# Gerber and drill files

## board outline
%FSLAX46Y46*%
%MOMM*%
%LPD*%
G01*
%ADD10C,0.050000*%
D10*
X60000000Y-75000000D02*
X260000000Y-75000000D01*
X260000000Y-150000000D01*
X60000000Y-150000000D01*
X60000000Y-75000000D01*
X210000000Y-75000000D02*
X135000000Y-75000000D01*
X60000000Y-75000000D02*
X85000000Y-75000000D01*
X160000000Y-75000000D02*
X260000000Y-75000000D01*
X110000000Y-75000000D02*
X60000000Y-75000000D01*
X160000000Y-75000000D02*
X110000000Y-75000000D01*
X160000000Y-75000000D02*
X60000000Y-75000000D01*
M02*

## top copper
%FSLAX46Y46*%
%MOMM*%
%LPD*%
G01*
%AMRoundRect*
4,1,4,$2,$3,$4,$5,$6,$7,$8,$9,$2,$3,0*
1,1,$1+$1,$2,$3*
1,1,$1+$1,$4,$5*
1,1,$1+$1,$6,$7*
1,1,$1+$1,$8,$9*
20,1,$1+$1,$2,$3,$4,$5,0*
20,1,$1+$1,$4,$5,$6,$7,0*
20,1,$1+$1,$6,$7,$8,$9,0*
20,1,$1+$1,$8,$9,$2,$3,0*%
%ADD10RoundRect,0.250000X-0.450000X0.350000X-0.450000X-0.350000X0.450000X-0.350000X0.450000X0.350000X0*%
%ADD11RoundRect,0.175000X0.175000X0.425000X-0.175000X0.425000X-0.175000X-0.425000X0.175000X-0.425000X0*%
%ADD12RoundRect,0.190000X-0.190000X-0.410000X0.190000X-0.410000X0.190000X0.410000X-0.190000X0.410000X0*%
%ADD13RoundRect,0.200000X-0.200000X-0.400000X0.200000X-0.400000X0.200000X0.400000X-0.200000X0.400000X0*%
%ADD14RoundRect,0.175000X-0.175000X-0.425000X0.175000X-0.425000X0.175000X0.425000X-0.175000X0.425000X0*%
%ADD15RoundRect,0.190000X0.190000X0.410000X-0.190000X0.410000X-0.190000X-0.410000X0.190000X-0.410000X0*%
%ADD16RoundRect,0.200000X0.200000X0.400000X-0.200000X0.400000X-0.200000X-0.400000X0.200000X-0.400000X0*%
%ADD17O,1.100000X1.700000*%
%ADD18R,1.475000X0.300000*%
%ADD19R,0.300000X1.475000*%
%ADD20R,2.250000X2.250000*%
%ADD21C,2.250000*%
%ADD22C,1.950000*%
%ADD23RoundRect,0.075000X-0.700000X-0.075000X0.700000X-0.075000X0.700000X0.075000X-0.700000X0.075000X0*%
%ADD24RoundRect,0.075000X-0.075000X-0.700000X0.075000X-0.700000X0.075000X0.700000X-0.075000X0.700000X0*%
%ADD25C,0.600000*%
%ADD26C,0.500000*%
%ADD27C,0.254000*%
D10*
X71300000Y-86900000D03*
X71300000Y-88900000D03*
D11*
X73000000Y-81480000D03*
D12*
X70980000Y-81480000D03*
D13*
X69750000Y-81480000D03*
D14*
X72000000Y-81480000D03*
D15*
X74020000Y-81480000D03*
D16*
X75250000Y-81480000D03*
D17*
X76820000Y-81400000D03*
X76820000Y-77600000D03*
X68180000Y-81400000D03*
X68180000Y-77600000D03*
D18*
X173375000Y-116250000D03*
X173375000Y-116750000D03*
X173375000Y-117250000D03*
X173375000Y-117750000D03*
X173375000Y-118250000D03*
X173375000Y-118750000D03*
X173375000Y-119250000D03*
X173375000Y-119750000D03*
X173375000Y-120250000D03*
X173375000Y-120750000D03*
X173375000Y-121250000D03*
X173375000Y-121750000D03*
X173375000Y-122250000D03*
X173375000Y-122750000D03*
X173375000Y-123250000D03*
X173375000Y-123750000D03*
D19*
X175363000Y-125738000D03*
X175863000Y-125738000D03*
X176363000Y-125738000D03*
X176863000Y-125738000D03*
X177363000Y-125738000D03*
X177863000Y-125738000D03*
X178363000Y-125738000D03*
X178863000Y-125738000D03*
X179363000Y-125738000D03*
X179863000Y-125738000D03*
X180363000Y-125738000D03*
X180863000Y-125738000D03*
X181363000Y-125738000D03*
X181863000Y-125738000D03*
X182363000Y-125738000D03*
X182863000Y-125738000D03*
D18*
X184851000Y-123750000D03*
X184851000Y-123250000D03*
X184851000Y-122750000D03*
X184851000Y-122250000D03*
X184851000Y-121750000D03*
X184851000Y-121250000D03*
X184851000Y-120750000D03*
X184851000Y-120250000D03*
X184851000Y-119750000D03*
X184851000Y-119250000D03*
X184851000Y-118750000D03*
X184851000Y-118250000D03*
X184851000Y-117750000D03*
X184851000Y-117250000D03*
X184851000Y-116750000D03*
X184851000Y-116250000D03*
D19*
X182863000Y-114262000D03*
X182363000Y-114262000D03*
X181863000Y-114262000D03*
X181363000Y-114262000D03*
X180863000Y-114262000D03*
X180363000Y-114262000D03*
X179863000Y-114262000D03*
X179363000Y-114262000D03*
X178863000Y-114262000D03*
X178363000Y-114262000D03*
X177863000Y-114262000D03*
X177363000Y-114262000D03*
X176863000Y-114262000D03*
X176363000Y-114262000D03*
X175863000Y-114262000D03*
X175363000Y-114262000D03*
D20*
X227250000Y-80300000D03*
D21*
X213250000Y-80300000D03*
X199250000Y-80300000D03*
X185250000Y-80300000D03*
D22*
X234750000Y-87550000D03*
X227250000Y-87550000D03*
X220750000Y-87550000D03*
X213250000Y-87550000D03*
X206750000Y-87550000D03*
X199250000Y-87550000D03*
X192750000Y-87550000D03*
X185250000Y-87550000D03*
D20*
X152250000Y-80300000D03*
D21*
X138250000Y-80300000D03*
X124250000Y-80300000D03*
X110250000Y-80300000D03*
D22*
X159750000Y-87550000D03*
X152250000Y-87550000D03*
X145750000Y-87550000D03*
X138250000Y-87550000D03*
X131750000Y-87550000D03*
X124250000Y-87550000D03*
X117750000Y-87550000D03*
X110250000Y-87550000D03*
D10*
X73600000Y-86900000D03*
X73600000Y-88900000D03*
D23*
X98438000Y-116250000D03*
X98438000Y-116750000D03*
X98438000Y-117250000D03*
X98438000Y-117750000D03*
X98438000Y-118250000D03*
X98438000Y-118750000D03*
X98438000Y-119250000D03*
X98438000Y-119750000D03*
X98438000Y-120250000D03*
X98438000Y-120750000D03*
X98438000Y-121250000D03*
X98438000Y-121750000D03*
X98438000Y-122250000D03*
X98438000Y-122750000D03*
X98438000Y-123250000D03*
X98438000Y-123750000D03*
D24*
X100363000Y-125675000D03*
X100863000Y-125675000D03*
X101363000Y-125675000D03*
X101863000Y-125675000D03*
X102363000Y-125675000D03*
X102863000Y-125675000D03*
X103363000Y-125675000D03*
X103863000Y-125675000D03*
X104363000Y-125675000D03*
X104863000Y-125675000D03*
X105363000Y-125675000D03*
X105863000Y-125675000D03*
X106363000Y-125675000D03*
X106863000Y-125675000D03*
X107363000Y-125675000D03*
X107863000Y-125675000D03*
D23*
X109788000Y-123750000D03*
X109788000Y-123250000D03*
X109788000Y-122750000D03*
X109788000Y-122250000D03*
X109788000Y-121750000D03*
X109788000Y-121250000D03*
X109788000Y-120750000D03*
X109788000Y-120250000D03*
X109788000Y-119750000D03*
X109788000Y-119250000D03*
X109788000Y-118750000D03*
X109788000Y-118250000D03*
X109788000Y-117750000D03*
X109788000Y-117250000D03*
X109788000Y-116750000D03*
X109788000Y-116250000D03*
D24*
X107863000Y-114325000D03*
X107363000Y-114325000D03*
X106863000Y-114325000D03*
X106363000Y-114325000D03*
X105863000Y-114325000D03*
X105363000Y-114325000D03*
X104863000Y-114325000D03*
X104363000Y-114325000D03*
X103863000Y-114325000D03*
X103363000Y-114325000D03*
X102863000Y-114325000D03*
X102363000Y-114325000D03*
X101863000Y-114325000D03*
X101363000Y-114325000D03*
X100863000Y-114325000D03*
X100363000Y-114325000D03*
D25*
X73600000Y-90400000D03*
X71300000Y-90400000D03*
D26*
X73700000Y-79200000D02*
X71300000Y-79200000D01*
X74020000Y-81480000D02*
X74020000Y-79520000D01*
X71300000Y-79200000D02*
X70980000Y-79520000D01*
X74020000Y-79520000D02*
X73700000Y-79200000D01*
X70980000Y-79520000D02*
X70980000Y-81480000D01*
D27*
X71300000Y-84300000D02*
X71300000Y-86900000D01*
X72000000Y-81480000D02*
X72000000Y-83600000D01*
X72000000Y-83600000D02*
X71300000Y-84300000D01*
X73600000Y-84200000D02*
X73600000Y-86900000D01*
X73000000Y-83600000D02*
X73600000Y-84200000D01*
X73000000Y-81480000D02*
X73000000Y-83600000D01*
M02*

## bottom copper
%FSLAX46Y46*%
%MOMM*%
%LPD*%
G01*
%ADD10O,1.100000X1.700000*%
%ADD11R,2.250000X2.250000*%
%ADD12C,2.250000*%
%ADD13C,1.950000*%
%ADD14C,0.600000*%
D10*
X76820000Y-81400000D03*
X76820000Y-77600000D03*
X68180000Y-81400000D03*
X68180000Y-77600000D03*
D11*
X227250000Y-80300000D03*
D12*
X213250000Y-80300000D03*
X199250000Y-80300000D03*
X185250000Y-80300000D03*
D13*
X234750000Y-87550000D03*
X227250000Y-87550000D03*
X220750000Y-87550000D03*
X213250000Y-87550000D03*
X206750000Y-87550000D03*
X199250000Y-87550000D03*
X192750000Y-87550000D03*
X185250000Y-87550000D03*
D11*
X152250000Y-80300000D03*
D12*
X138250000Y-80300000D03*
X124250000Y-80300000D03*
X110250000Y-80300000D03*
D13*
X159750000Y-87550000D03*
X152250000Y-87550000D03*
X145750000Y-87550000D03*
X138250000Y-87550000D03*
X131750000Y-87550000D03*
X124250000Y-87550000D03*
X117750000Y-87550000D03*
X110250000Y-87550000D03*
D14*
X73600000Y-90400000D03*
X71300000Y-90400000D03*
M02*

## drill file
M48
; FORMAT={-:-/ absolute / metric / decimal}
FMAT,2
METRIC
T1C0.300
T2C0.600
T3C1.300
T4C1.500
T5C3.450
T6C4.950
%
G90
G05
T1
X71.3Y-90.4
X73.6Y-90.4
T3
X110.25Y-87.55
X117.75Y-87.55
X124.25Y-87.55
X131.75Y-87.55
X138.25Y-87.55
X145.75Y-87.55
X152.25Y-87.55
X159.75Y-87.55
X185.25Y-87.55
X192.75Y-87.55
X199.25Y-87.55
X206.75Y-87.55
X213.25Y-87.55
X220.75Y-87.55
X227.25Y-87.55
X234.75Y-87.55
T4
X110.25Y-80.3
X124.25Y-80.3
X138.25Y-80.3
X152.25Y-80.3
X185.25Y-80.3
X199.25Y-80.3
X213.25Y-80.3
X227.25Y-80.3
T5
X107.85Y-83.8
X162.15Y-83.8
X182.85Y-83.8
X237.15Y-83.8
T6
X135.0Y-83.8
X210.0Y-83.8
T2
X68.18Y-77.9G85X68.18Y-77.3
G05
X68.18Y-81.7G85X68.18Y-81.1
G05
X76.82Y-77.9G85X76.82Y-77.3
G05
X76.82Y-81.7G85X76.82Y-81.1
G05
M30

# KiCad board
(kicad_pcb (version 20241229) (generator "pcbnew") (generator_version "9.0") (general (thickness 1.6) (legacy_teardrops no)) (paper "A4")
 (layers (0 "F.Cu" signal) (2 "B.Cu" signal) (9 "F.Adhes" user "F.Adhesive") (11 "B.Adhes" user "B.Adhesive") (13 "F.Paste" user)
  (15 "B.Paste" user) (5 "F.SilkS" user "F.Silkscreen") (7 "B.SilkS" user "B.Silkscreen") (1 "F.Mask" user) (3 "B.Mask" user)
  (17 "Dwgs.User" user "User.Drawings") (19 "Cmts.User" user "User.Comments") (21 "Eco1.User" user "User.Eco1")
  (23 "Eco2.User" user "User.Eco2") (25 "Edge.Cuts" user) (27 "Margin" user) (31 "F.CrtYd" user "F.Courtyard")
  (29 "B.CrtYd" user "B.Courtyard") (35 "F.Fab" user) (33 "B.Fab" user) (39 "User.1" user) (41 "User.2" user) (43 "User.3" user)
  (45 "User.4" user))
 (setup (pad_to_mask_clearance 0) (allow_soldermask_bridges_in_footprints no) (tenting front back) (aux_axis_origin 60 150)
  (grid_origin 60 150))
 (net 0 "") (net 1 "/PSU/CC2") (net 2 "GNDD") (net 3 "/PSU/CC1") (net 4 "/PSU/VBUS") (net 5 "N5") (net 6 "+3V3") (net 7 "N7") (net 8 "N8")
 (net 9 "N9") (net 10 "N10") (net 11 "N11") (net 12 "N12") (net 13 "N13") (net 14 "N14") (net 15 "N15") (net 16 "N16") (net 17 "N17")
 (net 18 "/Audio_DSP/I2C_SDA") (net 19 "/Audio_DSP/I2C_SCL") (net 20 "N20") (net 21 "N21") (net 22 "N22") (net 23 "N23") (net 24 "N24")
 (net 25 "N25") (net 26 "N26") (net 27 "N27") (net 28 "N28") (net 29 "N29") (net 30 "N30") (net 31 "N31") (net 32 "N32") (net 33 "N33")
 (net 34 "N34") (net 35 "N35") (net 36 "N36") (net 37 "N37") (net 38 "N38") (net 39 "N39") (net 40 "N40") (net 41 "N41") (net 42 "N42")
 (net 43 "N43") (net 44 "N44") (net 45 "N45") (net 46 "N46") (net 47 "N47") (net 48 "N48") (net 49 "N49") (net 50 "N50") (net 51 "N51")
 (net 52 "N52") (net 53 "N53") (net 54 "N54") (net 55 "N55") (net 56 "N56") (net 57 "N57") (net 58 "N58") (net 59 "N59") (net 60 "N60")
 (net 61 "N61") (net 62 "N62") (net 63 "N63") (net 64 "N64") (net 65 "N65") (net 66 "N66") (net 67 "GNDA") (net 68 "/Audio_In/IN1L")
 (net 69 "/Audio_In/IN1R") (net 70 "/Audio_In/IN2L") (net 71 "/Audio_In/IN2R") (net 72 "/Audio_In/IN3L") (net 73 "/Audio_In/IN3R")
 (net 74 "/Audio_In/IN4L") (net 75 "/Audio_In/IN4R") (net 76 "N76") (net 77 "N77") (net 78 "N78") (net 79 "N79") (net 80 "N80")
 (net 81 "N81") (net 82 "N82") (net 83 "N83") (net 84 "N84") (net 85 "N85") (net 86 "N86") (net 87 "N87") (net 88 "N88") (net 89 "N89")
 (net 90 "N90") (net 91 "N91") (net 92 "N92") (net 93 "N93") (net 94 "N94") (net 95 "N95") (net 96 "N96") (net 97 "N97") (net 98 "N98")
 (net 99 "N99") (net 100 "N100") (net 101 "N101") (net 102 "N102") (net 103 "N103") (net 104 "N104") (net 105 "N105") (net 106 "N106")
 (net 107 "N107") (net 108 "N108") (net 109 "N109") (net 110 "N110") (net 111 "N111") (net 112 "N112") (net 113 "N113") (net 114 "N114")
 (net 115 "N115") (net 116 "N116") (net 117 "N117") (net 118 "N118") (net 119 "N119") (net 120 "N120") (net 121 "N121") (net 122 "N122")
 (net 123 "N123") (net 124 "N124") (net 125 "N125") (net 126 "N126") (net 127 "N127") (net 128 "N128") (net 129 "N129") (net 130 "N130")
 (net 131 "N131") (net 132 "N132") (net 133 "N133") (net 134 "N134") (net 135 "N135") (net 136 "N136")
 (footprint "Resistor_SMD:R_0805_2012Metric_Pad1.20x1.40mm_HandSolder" (layer "F.Cu") (at 71.3 87.9 -90)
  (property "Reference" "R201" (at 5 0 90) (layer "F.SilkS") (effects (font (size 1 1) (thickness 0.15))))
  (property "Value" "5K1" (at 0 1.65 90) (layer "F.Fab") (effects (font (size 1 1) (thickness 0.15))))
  (pad "1" smd roundrect (at -1 0 270) (size 1.2 1.4) (layers "F.Cu" "F.Mask" "F.Paste") (roundrect_rratio 0.208333) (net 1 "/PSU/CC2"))
  (pad "2" smd roundrect (at 1 0 270) (size 1.2 1.4) (layers "F.Cu" "F.Mask" "F.Paste") (roundrect_rratio 0.208333) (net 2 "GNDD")))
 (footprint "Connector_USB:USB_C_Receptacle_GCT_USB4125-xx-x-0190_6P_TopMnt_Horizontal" (layer "F.Cu") (at 72.5 78.4 180)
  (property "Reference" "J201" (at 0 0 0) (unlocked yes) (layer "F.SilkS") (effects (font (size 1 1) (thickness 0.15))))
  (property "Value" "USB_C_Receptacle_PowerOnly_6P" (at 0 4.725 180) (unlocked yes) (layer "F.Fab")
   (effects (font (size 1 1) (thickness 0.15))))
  (pad "A5" smd roundrect (at -0.5 -3.08 180) (size 0.7 1.2) (layers "F.Cu" "F.Mask" "F.Paste") (roundrect_rratio 0.25) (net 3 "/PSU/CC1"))
  (pad "A9" smd roundrect (at 1.52 -3.08) (size 0.76 1.2) (layers "F.Cu" "F.Mask" "F.Paste") (roundrect_rratio 0.25) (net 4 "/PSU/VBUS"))
  (pad "A12" smd roundrect (at 2.75 -3.08) (size 0.8 1.2) (layers "F.Cu" "F.Mask" "F.Paste") (roundrect_rratio 0.25) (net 2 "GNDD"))
  (pad "B5" smd roundrect (at 0.5 -3.08) (size 0.7 1.2) (layers "F.Cu" "F.Mask" "F.Paste") (roundrect_rratio 0.25) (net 1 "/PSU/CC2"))
  (pad "B9" smd roundrect (at -1.52 -3.08 180) (size 0.76 1.2) (layers "F.Cu" "F.Mask" "F.Paste") (roundrect_rratio 0.25)
   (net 4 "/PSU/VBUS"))
  (pad "B12" smd roundrect (at -2.75 -3.08 180) (size 0.8 1.2) (layers "F.Cu" "F.Mask" "F.Paste") (roundrect_rratio 0.25) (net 2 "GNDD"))
  (pad "S1" thru_hole oval (at -4.32 -3 180) (size 1.1 1.7) (drill oval 0.6 1.2) (layers "*.Cu" "*.Mask" "F.Paste")
   (remove_unused_layers no) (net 2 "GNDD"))
  (pad "S1" thru_hole oval (at -4.32 0.8 180) (size 1.1 1.7) (drill oval 0.6 1.2) (layers "*.Cu" "*.Mask" "F.Paste")
   (remove_unused_layers no) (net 2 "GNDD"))
  (pad "S1" thru_hole oval (at 4.32 -3 180) (size 1.1 1.7) (drill oval 0.6 1.2) (layers "*.Cu" "*.Mask" "F.Paste") (remove_unused_layers no)
   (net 2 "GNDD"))
  (pad "S1" thru_hole oval (at 4.32 0.8 180) (size 1.1 1.7) (drill oval 0.6 1.2) (layers "*.Cu" "*.Mask" "F.Paste")
   (remove_unused_layers no) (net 2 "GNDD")))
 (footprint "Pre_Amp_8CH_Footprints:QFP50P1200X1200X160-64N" (layer "F.Cu") (at 179.113 120)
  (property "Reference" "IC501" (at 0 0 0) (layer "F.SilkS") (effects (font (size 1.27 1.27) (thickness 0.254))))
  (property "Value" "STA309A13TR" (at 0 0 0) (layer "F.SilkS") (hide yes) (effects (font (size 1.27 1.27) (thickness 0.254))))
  (pad "1" smd rect (at -5.738 -3.75 90) (size 0.3 1.475) (layers "F.Cu" "F.Mask" "F.Paste") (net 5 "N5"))
  (pad "2" smd rect (at -5.738 -3.25 90) (size 0.3 1.475) (layers "F.Cu" "F.Mask" "F.Paste") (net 2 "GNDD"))
  (pad "3" smd rect (at -5.738 -2.75 90) (size 0.3 1.475) (layers "F.Cu" "F.Mask" "F.Paste") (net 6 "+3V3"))
  (pad "4" smd rect (at -5.738 -2.25 90) (size 0.3 1.475) (layers "F.Cu" "F.Mask" "F.Paste") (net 2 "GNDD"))
  (pad "5" smd rect (at -5.738 -1.75 90) (size 0.3 1.475) (layers "F.Cu" "F.Mask" "F.Paste") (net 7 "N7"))
  (pad "6" smd rect (at -5.738 -1.25 90) (size 0.3 1.475) (layers "F.Cu" "F.Mask" "F.Paste") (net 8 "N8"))
  (pad "7" smd rect (at -5.738 -0.75 90) (size 0.3 1.475) (layers "F.Cu" "F.Mask" "F.Paste") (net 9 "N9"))
  (pad "8" smd rect (at -5.738 -0.25 90) (size 0.3 1.475) (layers "F.Cu" "F.Mask" "F.Paste") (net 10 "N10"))
  (pad "9" smd rect (at -5.738 0.25 90) (size 0.3 1.475) (layers "F.Cu" "F.Mask" "F.Paste") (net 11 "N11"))
  (pad "10" smd rect (at -5.738 0.75 90) (size 0.3 1.475) (layers "F.Cu" "F.Mask" "F.Paste") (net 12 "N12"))
  (pad "11" smd rect (at -5.738 1.25 90) (size 0.3 1.475) (layers "F.Cu" "F.Mask" "F.Paste") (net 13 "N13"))
  (pad "12" smd rect (at -5.738 1.75 90) (size 0.3 1.475) (layers "F.Cu" "F.Mask" "F.Paste") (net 6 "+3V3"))
  (pad "13" smd rect (at -5.738 2.25 90) (size 0.3 1.475) (layers "F.Cu" "F.Mask" "F.Paste") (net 2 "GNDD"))
  (pad "14" smd rect (at -5.738 2.75 90) (size 0.3 1.475) (layers "F.Cu" "F.Mask" "F.Paste") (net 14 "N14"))
  (pad "15" smd rect (at -5.738 3.25 90) (size 0.3 1.475) (layers "F.Cu" "F.Mask" "F.Paste") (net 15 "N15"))
  (pad "16" smd rect (at -5.738 3.75 90) (size 0.3 1.475) (layers "F.Cu" "F.Mask" "F.Paste") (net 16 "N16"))
  (pad "17" smd rect (at -3.75 5.738) (size 0.3 1.475) (layers "F.Cu" "F.Mask" "F.Paste") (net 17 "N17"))
  (pad "18" smd rect (at -3.25 5.738) (size 0.3 1.475) (layers "F.Cu" "F.Mask" "F.Paste") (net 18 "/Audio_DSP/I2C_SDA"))
  (pad "19" smd rect (at -2.75 5.738) (size 0.3 1.475) (layers "F.Cu" "F.Mask" "F.Paste") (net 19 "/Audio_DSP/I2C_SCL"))
  (pad "20" smd rect (at -2.25 5.738) (size 0.3 1.475) (layers "F.Cu" "F.Mask" "F.Paste") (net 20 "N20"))
  (pad "21" smd rect (at -1.75 5.738) (size 0.3 1.475) (layers "F.Cu" "F.Mask" "F.Paste") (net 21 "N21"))
  (pad "22" smd rect (at -1.25 5.738) (size 0.3 1.475) (layers "F.Cu" "F.Mask" "F.Paste") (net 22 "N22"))
  (pad "23" smd rect (at -0.75 5.738) (size 0.3 1.475) (layers "F.Cu" "F.Mask" "F.Paste") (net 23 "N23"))
  (pad "24" smd rect (at -0.25 5.738) (size 0.3 1.475) (layers "F.Cu" "F.Mask" "F.Paste") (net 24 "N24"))
  (pad "25" smd rect (at 0.25 5.738) (size 0.3 1.475) (layers "F.Cu" "F.Mask" "F.Paste") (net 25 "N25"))
  (pad "26" smd rect (at 0.75 5.738) (size 0.3 1.475) (layers "F.Cu" "F.Mask" "F.Paste") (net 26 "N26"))
  (pad "27" smd rect (at 1.25 5.738) (size 0.3 1.475) (layers "F.Cu" "F.Mask" "F.Paste") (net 2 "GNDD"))
  (pad "28" smd rect (at 1.75 5.738) (size 0.3 1.475) (layers "F.Cu" "F.Mask" "F.Paste") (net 6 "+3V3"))
  (pad "29" smd rect (at 2.25 5.738) (size 0.3 1.475) (layers "F.Cu" "F.Mask" "F.Paste") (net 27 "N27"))
  (pad "30" smd rect (at 2.75 5.738) (size 0.3 1.475) (layers "F.Cu" "F.Mask" "F.Paste") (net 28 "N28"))
  (pad "31" smd rect (at 3.25 5.738) (size 0.3 1.475) (layers "F.Cu" "F.Mask" "F.Paste") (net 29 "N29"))
  (pad "32" smd rect (at 3.75 5.738) (size 0.3 1.475) (layers "F.Cu" "F.Mask" "F.Paste") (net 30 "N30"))
  (pad "33" smd rect (at 5.738 3.75 90) (size 0.3 1.475) (layers "F.Cu" "F.Mask" "F.Paste") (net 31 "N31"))
  (pad "34" smd rect (at 5.738 3.25 90) (size 0.3 1.475) (layers "F.Cu" "F.Mask" "F.Paste") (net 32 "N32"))
  (pad "35" smd rect (at 5.738 2.75 90) (size 0.3 1.475) (layers "F.Cu" "F.Mask" "F.Paste") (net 6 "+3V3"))
  (pad "36" smd rect (at 5.738 2.25 90) (size 0.3 1.475) (layers "F.Cu" "F.Mask" "F.Paste") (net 2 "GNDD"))
  (pad "37" smd rect (at 5.738 1.75 90) (size 0.3 1.475) (layers "F.Cu" "F.Mask" "F.Paste") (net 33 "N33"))
  (pad "38" smd rect (at 5.738 1.25 90) (size 0.3 1.475) (layers "F.Cu" "F.Mask" "F.Paste") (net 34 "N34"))
  (pad "39" smd rect (at 5.738 0.75 90) (size 0.3 1.475) (layers "F.Cu" "F.Mask" "F.Paste") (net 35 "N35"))
  (pad "40" smd rect (at 5.738 0.25 90) (size 0.3 1.475) (layers "F.Cu" "F.Mask" "F.Paste") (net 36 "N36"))
  (pad "41" smd rect (at 5.738 -0.25 90) (size 0.3 1.475) (layers "F.Cu" "F.Mask" "F.Paste") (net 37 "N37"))
  (pad "42" smd rect (at 5.738 -0.75 90) (size 0.3 1.475) (layers "F.Cu" "F.Mask" "F.Paste") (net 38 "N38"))
  (pad "43" smd rect (at 5.738 -1.25 90) (size 0.3 1.475) (layers "F.Cu" "F.Mask" "F.Paste") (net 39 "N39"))
  (pad "44" smd rect (at 5.738 -1.75 90) (size 0.3 1.475) (layers "F.Cu" "F.Mask" "F.Paste") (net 6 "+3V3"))
  (pad "45" smd rect (at 5.738 -2.25 90) (size 0.3 1.475) (layers "F.Cu" "F.Mask" "F.Paste") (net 2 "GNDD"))
  (pad "46" smd rect (at 5.738 -2.75 90) (size 0.3 1.475) (layers "F.Cu" "F.Mask" "F.Paste") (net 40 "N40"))
  (pad "47" smd rect (at 5.738 -3.25 90) (size 0.3 1.475) (layers "F.Cu" "F.Mask" "F.Paste") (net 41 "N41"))
  (pad "48" smd rect (at 5.738 -3.75 90) (size 0.3 1.475) (layers "F.Cu" "F.Mask" "F.Paste") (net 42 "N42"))
  (pad "49" smd rect (at 3.75 -5.738) (size 0.3 1.475) (layers "F.Cu" "F.Mask" "F.Paste") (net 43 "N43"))
  (pad "50" smd rect (at 3.25 -5.738) (size 0.3 1.475) (layers "F.Cu" "F.Mask" "F.Paste") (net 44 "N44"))
  (pad "51" smd rect (at 2.75 -5.738) (size 0.3 1.475) (layers "F.Cu" "F.Mask" "F.Paste") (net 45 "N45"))
  (pad "52" smd rect (at 2.25 -5.738) (size 0.3 1.475) (layers "F.Cu" "F.Mask" "F.Paste") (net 6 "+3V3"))
  (pad "53" smd rect (at 1.75 -5.738) (size 0.3 1.475) (layers "F.Cu" "F.Mask" "F.Paste") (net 2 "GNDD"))
  (pad "54" smd rect (at 1.25 -5.738) (size 0.3 1.475) (layers "F.Cu" "F.Mask" "F.Paste") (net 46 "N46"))
  (pad "55" smd rect (at 0.75 -5.738) (size 0.3 1.475) (layers "F.Cu" "F.Mask" "F.Paste") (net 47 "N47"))
  (pad "56" smd rect (at 0.25 -5.738) (size 0.3 1.475) (layers "F.Cu" "F.Mask" "F.Paste") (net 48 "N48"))
  (pad "57" smd rect (at -0.25 -5.738) (size 0.3 1.475) (layers "F.Cu" "F.Mask" "F.Paste") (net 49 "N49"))
  (pad "58" smd rect (at -0.75 -5.738) (size 0.3 1.475) (layers "F.Cu" "F.Mask" "F.Paste") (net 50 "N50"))
  (pad "59" smd rect (at -1.25 -5.738) (size 0.3 1.475) (layers "F.Cu" "F.Mask" "F.Paste") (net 6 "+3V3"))
  (pad "60" smd rect (at -1.75 -5.738) (size 0.3 1.475) (layers "F.Cu" "F.Mask" "F.Paste") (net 2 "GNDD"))
  (pad "61" smd rect (at -2.25 -5.738) (size 0.3 1.475) (layers "F.Cu" "F.Mask" "F.Paste") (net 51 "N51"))
  (pad "62" smd rect (at -2.75 -5.738) (size 0.3 1.475) (layers "F.Cu" "F.Mask" "F.Paste") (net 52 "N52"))
  (pad "63" smd rect (at -3.25 -5.738) (size 0.3 1.475) (layers "F.Cu" "F.Mask" "F.Paste") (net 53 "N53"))
  (pad "64" smd rect (at -3.75 -5.738) (size 0.3 1.475) (layers "F.Cu" "F.Mask" "F.Paste") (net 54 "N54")))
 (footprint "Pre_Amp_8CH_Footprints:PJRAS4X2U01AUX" (layer "F.Cu") (at 227.25 80.3 180)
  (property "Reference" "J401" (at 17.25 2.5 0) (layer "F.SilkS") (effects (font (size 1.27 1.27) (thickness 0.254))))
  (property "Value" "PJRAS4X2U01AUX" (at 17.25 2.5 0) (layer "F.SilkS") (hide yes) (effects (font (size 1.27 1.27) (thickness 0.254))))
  (pad "" np_thru_hole circle (at -9.9 -3.5 180) (size 3.45 3.45) (drill 3.45) (layers "*.Cu" "*.Mask"))
  (pad "" np_thru_hole circle (at 17.25 -3.5 180) (size 4.95 4.95) (drill 4.95) (layers "*.Cu" "*.Mask"))
  (pad "" np_thru_hole circle (at 44.4 -3.5 180) (size 3.45 3.45) (drill 3.45) (layers "*.Cu" "*.Mask"))
  (pad "S1" thru_hole rect (at 0 0 180) (size 2.25 2.25) (drill 1.5) (layers "*.Cu" "*.Mask") (remove_unused_layers no) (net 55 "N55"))
  (pad "S2" thru_hole circle (at 14 0 180) (size 2.25 2.25) (drill 1.5) (layers "*.Cu" "*.Mask") (remove_unused_layers no) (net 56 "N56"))
  (pad "S3" thru_hole circle (at 28 0 180) (size 2.25 2.25) (drill 1.5) (layers "*.Cu" "*.Mask") (remove_unused_layers no) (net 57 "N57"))
  (pad "S4" thru_hole circle (at 42 0 180) (size 2.25 2.25) (drill 1.5) (layers "*.Cu" "*.Mask") (remove_unused_layers no) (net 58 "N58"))
  (pad "T11" thru_hole circle (at -7.5 -7.25 180) (size 1.95 1.95) (drill 1.3) (layers "*.Cu" "*.Mask") (remove_unused_layers no)
   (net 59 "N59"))
  (pad "T12" thru_hole circle (at 0 -7.25 180) (size 1.95 1.95) (drill 1.3) (layers "*.Cu" "*.Mask") (remove_unused_layers no)
   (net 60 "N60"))
  (pad "T21" thru_hole circle (at 6.5 -7.25 180) (size 1.95 1.95) (drill 1.3) (layers "*.Cu" "*.Mask") (remove_unused_layers no)
   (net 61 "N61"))
  (pad "T22" thru_hole circle (at 14 -7.25 180) (size 1.95 1.95) (drill 1.3) (layers "*.Cu" "*.Mask") (remove_unused_layers no)
   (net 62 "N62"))
  (pad "T31" thru_hole circle (at 20.5 -7.25 180) (size 1.95 1.95) (drill 1.3) (layers "*.Cu" "*.Mask") (remove_unused_layers no)
   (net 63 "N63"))
  (pad "T32" thru_hole circle (at 28 -7.25 180) (size 1.95 1.95) (drill 1.3) (layers "*.Cu" "*.Mask") (remove_unused_layers no)
   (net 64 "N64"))
  (pad "T41" thru_hole circle (at 34.5 -7.25 180) (size 1.95 1.95) (drill 1.3) (layers "*.Cu" "*.Mask") (remove_unused_layers no)
   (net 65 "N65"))
  (pad "T42" thru_hole circle (at 42 -7.25 180) (size 1.95 1.95) (drill 1.3) (layers "*.Cu" "*.Mask") (remove_unused_layers no)
   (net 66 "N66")))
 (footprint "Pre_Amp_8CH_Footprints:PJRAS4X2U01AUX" (layer "F.Cu") (at 152.25 80.3 180)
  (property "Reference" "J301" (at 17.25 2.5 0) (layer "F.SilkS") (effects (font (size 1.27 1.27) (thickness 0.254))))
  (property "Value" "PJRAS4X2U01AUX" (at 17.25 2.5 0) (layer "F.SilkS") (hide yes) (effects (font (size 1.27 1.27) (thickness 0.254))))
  (pad "" np_thru_hole circle (at -9.9 -3.5 180) (size 3.45 3.45) (drill 3.45) (layers "*.Cu" "*.Mask"))
  (pad "" np_thru_hole circle (at 17.25 -3.5 180) (size 4.95 4.95) (drill 4.95) (layers "*.Cu" "*.Mask"))
  (pad "" np_thru_hole circle (at 44.4 -3.5 180) (size 3.45 3.45) (drill 3.45) (layers "*.Cu" "*.Mask"))
  (pad "S1" thru_hole rect (at 0 0 180) (size 2.25 2.25) (drill 1.5) (layers "*.Cu" "*.Mask") (remove_unused_layers no) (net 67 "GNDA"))
  (pad "S2" thru_hole circle (at 14 0 180) (size 2.25 2.25) (drill 1.5) (layers "*.Cu" "*.Mask") (remove_unused_layers no) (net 67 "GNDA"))
  (pad "S3" thru_hole circle (at 28 0 180) (size 2.25 2.25) (drill 1.5) (layers "*.Cu" "*.Mask") (remove_unused_layers no) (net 67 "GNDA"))
  (pad "S4" thru_hole circle (at 42 0 180) (size 2.25 2.25) (drill 1.5) (layers "*.Cu" "*.Mask") (remove_unused_layers no) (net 67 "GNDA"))
  (pad "T11" thru_hole circle (at -7.5 -7.25 180) (size 1.95 1.95) (drill 1.3) (layers "*.Cu" "*.Mask") (remove_unused_layers no)
   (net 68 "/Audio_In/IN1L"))
  (pad "T12" thru_hole circle (at 0 -7.25 180) (size 1.95 1.95) (drill 1.3) (layers "*.Cu" "*.Mask") (remove_unused_layers no)
   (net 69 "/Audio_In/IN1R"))
  (pad "T21" thru_hole circle (at 6.5 -7.25 180) (size 1.95 1.95) (drill 1.3) (layers "*.Cu" "*.Mask") (remove_unused_layers no)
   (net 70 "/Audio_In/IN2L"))
  (pad "T22" thru_hole circle (at 14 -7.25 180) (size 1.95 1.95) (drill 1.3) (layers "*.Cu" "*.Mask") (remove_unused_layers no)
   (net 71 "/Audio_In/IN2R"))
  (pad "T31" thru_hole circle (at 20.5 -7.25 180) (size 1.95 1.95) (drill 1.3) (layers "*.Cu" "*.Mask") (remove_unused_layers no)
   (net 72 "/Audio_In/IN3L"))
  (pad "T32" thru_hole circle (at 28 -7.25 180) (size 1.95 1.95) (drill 1.3) (layers "*.Cu" "*.Mask") (remove_unused_layers no)
   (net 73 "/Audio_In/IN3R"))
  (pad "T41" thru_hole circle (at 34.5 -7.25 180) (size 1.95 1.95) (drill 1.3) (layers "*.Cu" "*.Mask") (remove_unused_layers no)
   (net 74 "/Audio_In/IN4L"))
  (pad "T42" thru_hole circle (at 42 -7.25 180) (size 1.95 1.95) (drill 1.3) (layers "*.Cu" "*.Mask") (remove_unused_layers no)
   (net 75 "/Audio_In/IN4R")))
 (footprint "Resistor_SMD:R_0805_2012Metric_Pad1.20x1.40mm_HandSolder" (layer "F.Cu") (at 73.6 87.9 -90)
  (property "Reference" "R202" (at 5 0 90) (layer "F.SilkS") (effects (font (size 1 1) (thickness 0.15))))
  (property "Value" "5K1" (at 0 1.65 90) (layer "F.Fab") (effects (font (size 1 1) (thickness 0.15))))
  (pad "1" smd roundrect (at -1 0 270) (size 1.2 1.4) (layers "F.Cu" "F.Mask" "F.Paste") (roundrect_rratio 0.208333) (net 3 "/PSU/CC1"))
  (pad "2" smd roundrect (at 1 0 270) (size 1.2 1.4) (layers "F.Cu" "F.Mask" "F.Paste") (roundrect_rratio 0.208333) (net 2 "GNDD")))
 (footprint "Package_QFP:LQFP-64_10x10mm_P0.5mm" (layer "F.Cu") (at 104.113 120)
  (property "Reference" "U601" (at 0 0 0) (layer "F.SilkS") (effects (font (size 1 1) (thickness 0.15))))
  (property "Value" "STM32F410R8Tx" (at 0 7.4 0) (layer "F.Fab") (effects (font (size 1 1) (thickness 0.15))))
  (pad "1" smd roundrect (at -5.675 -3.75) (size 1.55 0.3) (layers "F.Cu" "F.Mask" "F.Paste") (roundrect_rratio 0.25) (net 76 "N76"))
  (pad "2" smd roundrect (at -5.675 -3.25) (size 1.55 0.3) (layers "F.Cu" "F.Mask" "F.Paste") (roundrect_rratio 0.25) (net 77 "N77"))
  (pad "3" smd roundrect (at -5.675 -2.75) (size 1.55 0.3) (layers "F.Cu" "F.Mask" "F.Paste") (roundrect_rratio 0.25) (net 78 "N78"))
  (pad "4" smd roundrect (at -5.675 -2.25) (size 1.55 0.3) (layers "F.Cu" "F.Mask" "F.Paste") (roundrect_rratio 0.25) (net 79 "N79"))
  (pad "5" smd roundrect (at -5.675 -1.75) (size 1.55 0.3) (layers "F.Cu" "F.Mask" "F.Paste") (roundrect_rratio 0.25) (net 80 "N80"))
  (pad "6" smd roundrect (at -5.675 -1.25) (size 1.55 0.3) (layers "F.Cu" "F.Mask" "F.Paste") (roundrect_rratio 0.25) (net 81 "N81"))
  (pad "7" smd roundrect (at -5.675 -0.75) (size 1.55 0.3) (layers "F.Cu" "F.Mask" "F.Paste") (roundrect_rratio 0.25) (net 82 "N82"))
  (pad "8" smd roundrect (at -5.675 -0.25) (size 1.55 0.3) (layers "F.Cu" "F.Mask" "F.Paste") (roundrect_rratio 0.25) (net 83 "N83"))
  (pad "9" smd roundrect (at -5.675 0.25) (size 1.55 0.3) (layers "F.Cu" "F.Mask" "F.Paste") (roundrect_rratio 0.25) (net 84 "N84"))
  (pad "10" smd roundrect (at -5.675 0.75) (size 1.55 0.3) (layers "F.Cu" "F.Mask" "F.Paste") (roundrect_rratio 0.25) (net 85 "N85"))
  (pad "11" smd roundrect (at -5.675 1.25) (size 1.55 0.3) (layers "F.Cu" "F.Mask" "F.Paste") (roundrect_rratio 0.25) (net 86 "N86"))
  (pad "12" smd roundrect (at -5.675 1.75) (size 1.55 0.3) (layers "F.Cu" "F.Mask" "F.Paste") (roundrect_rratio 0.25) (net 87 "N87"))
  (pad "13" smd roundrect (at -5.675 2.25) (size 1.55 0.3) (layers "F.Cu" "F.Mask" "F.Paste") (roundrect_rratio 0.25) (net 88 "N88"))
  (pad "14" smd roundrect (at -5.675 2.75) (size 1.55 0.3) (layers "F.Cu" "F.Mask" "F.Paste") (roundrect_rratio 0.25) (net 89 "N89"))
  (pad "15" smd roundrect (at -5.675 3.25) (size 1.55 0.3) (layers "F.Cu" "F.Mask" "F.Paste") (roundrect_rratio 0.25) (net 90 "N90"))
  (pad "16" smd roundrect (at -5.675 3.75) (size 1.55 0.3) (layers "F.Cu" "F.Mask" "F.Paste") (roundrect_rratio 0.25) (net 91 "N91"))
  (pad "17" smd roundrect (at -3.75 5.675) (size 0.3 1.55) (layers "F.Cu" "F.Mask" "F.Paste") (roundrect_rratio 0.25) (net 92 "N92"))
  (pad "18" smd roundrect (at -3.25 5.675) (size 0.3 1.55) (layers "F.Cu" "F.Mask" "F.Paste") (roundrect_rratio 0.25) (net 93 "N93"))
  (pad "19" smd roundrect (at -2.75 5.675) (size 0.3 1.55) (layers "F.Cu" "F.Mask" "F.Paste") (roundrect_rratio 0.25) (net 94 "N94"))
  (pad "20" smd roundrect (at -2.25 5.675) (size 0.3 1.55) (layers "F.Cu" "F.Mask" "F.Paste") (roundrect_rratio 0.25) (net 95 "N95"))
  (pad "21" smd roundrect (at -1.75 5.675) (size 0.3 1.55) (layers "F.Cu" "F.Mask" "F.Paste") (roundrect_rratio 0.25) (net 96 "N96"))
  (pad "22" smd roundrect (at -1.25 5.675) (size 0.3 1.55) (layers "F.Cu" "F.Mask" "F.Paste") (roundrect_rratio 0.25) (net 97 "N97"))
  (pad "23" smd roundrect (at -0.75 5.675) (size 0.3 1.55) (layers "F.Cu" "F.Mask" "F.Paste") (roundrect_rratio 0.25) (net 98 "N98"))
  (pad "24" smd roundrect (at -0.25 5.675) (size 0.3 1.55) (layers "F.Cu" "F.Mask" "F.Paste") (roundrect_rratio 0.25) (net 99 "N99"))
  (pad "25" smd roundrect (at 0.25 5.675) (size 0.3 1.55) (layers "F.Cu" "F.Mask" "F.Paste") (roundrect_rratio 0.25) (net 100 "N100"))
  (pad "26" smd roundrect (at 0.75 5.675) (size 0.3 1.55) (layers "F.Cu" "F.Mask" "F.Paste") (roundrect_rratio 0.25) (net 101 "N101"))
  (pad "27" smd roundrect (at 1.25 5.675) (size 0.3 1.55) (layers "F.Cu" "F.Mask" "F.Paste") (roundrect_rratio 0.25) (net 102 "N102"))
  (pad "28" smd roundrect (at 1.75 5.675) (size 0.3 1.55) (layers "F.Cu" "F.Mask" "F.Paste") (roundrect_rratio 0.25) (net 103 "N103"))
  (pad "29" smd roundrect (at 2.25 5.675) (size 0.3 1.55) (layers "F.Cu" "F.Mask" "F.Paste") (roundrect_rratio 0.25) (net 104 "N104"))
  (pad "30" smd roundrect (at 2.75 5.675) (size 0.3 1.55) (layers "F.Cu" "F.Mask" "F.Paste") (roundrect_rratio 0.25) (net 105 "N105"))
  (pad "31" smd roundrect (at 3.25 5.675) (size 0.3 1.55) (layers "F.Cu" "F.Mask" "F.Paste") (roundrect_rratio 0.25) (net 93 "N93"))
  (pad "32" smd roundrect (at 3.75 5.675) (size 0.3 1.55) (layers "F.Cu" "F.Mask" "F.Paste") (roundrect_rratio 0.25) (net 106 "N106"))
  (pad "33" smd roundrect (at 5.675 3.75) (size 1.55 0.3) (layers "F.Cu" "F.Mask" "F.Paste") (roundrect_rratio 0.25) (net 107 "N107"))
  (pad "34" smd roundrect (at 5.675 3.25) (size 1.55 0.3) (layers "F.Cu" "F.Mask" "F.Paste") (roundrect_rratio 0.25) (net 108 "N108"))
  (pad "35" smd roundrect (at 5.675 2.75) (size 1.55 0.3) (layers "F.Cu" "F.Mask" "F.Paste") (roundrect_rratio 0.25) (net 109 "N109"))
  (pad "36" smd roundrect (at 5.675 2.25) (size 1.55 0.3) (layers "F.Cu" "F.Mask" "F.Paste") (roundrect_rratio 0.25) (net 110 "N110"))
  (pad "37" smd roundrect (at 5.675 1.75) (size 1.55 0.3) (layers "F.Cu" "F.Mask" "F.Paste") (roundrect_rratio 0.25) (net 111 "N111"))
  (pad "38" smd roundrect (at 5.675 1.25) (size 1.55 0.3) (layers "F.Cu" "F.Mask" "F.Paste") (roundrect_rratio 0.25) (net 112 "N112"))
  (pad "39" smd roundrect (at 5.675 0.75) (size 1.55 0.3) (layers "F.Cu" "F.Mask" "F.Paste") (roundrect_rratio 0.25) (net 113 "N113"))
  (pad "40" smd roundrect (at 5.675 0.25) (size 1.55 0.3) (layers "F.Cu" "F.Mask" "F.Paste") (roundrect_rratio 0.25) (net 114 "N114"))
  (pad "41" smd roundrect (at 5.675 -0.25) (size 1.55 0.3) (layers "F.Cu" "F.Mask" "F.Paste") (roundrect_rratio 0.25) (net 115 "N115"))
  (pad "42" smd roundrect (at 5.675 -0.75) (size 1.55 0.3) (layers "F.Cu" "F.Mask" "F.Paste") (roundrect_rratio 0.25) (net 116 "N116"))
  (pad "43" smd roundrect (at 5.675 -1.25) (size 1.55 0.3) (layers "F.Cu" "F.Mask" "F.Paste") (roundrect_rratio 0.25) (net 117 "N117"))
  (pad "44" smd roundrect (at 5.675 -1.75) (size 1.55 0.3) (layers "F.Cu" "F.Mask" "F.Paste") (roundrect_rratio 0.25) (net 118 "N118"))
  (pad "45" smd roundrect (at 5.675 -2.25) (size 1.55 0.3) (layers "F.Cu" "F.Mask" "F.Paste") (roundrect_rratio 0.25) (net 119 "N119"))
  (pad "46" smd roundrect (at 5.675 -2.75) (size 1.55 0.3) (layers "F.Cu" "F.Mask" "F.Paste") (roundrect_rratio 0.25) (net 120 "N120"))
  (pad "47" smd roundrect (at 5.675 -3.25) (size 1.55 0.3) (layers "F.Cu" "F.Mask" "F.Paste") (roundrect_rratio 0.25) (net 93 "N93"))
  (pad "48" smd roundrect (at 5.675 -3.75) (size 1.55 0.3) (layers "F.Cu" "F.Mask" "F.Paste") (roundrect_rratio 0.25) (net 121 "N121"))
  (pad "49" smd roundrect (at 3.75 -5.675) (size 0.3 1.55) (layers "F.Cu" "F.Mask" "F.Paste") (roundrect_rratio 0.25) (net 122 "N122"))
  (pad "50" smd roundrect (at 3.25 -5.675) (size 0.3 1.55) (layers "F.Cu" "F.Mask" "F.Paste") (roundrect_rratio 0.25) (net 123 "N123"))
  (pad "51" smd roundrect (at 2.75 -5.675) (size 0.3 1.55) (layers "F.Cu" "F.Mask" "F.Paste") (roundrect_rratio 0.25) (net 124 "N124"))
  (pad "52" smd roundrect (at 2.25 -5.675) (size 0.3 1.55) (layers "F.Cu" "F.Mask" "F.Paste") (roundrect_rratio 0.25) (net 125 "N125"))
  (pad "53" smd roundrect (at 1.75 -5.675) (size 0.3 1.55) (layers "F.Cu" "F.Mask" "F.Paste") (roundrect_rratio 0.25) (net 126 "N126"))
  (pad "54" smd roundrect (at 1.25 -5.675) (size 0.3 1.55) (layers "F.Cu" "F.Mask" "F.Paste") (roundrect_rratio 0.25) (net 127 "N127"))
  (pad "55" smd roundrect (at 0.75 -5.675) (size 0.3 1.55) (layers "F.Cu" "F.Mask" "F.Paste") (roundrect_rratio 0.25) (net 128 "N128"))
  (pad "56" smd roundrect (at 0.25 -5.675) (size 0.3 1.55) (layers "F.Cu" "F.Mask" "F.Paste") (roundrect_rratio 0.25) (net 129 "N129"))
  (pad "57" smd roundrect (at -0.25 -5.675) (size 0.3 1.55) (layers "F.Cu" "F.Mask" "F.Paste") (roundrect_rratio 0.25) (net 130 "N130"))
  (pad "58" smd roundrect (at -0.75 -5.675) (size 0.3 1.55) (layers "F.Cu" "F.Mask" "F.Paste") (roundrect_rratio 0.25) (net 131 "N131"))
  (pad "59" smd roundrect (at -1.25 -5.675) (size 0.3 1.55) (layers "F.Cu" "F.Mask" "F.Paste") (roundrect_rratio 0.25) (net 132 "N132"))
  (pad "60" smd roundrect (at -1.75 -5.675) (size 0.3 1.55) (layers "F.Cu" "F.Mask" "F.Paste") (roundrect_rratio 0.25) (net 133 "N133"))
  (pad "61" smd roundrect (at -2.25 -5.675) (size 0.3 1.55) (layers "F.Cu" "F.Mask" "F.Paste") (roundrect_rratio 0.25) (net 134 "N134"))
  (pad "62" smd roundrect (at -2.75 -5.675) (size 0.3 1.55) (layers "F.Cu" "F.Mask" "F.Paste") (roundrect_rratio 0.25) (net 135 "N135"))
  (pad "63" smd roundrect (at -3.25 -5.675) (size 0.3 1.55) (layers "F.Cu" "F.Mask" "F.Paste") (roundrect_rratio 0.25) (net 93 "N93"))
  (pad "64" smd roundrect (at -3.75 -5.675) (size 0.3 1.55) (layers "F.Cu" "F.Mask" "F.Paste") (roundrect_rratio 0.25) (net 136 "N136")))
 (gr_rect (start 60 75) (end 260 150) (stroke (width 0.05) (type solid)) (fill no) (layer "Edge.Cuts"))
 (gr_line (start 210 75) (end 135 75) (stroke (width 0.05) (type default)) (layer "Edge.Cuts"))
 (gr_line (start 60 75) (end 85 75) (stroke (width 0.05) (type default)) (layer "Edge.Cuts"))
 (gr_line (start 160 75) (end 260 75) (stroke (width 0.05) (type default)) (layer "Edge.Cuts"))
 (gr_line (start 110 75) (end 60 75) (stroke (width 0.05) (type default)) (layer "Edge.Cuts"))
 (gr_line (start 160 75) (end 110 75) (stroke (width 0.05) (type default)) (layer "Edge.Cuts"))
 (gr_line (start 160 75) (end 60 75) (stroke (width 0.05) (type default)) (layer "Edge.Cuts"))
 (via (at 73.6 90.4) (size 0.6) (drill 0.3) (layers "F.Cu" "B.Cu") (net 2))
 (via (at 71.3 90.4) (size 0.6) (drill 0.3) (layers "F.Cu" "B.Cu") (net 2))
 (segment (start 73.7 79.2) (end 71.3 79.2) (width 0.5) (layer "F.Cu") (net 4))
 (segment (start 74.02 81.48) (end 74.02 79.52) (width 0.5) (layer "F.Cu") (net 4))
 (segment (start 71.3 79.2) (end 70.98 79.52) (width 0.5) (layer "F.Cu") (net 4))
 (segment (start 74.02 79.52) (end 73.7 79.2) (width 0.5) (layer "F.Cu") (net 4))
 (segment (start 70.98 79.52) (end 70.98 81.48) (width 0.5) (layer "F.Cu") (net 4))
 (segment (start 71.3 84.3) (end 71.3 86.9) (width 0.254) (layer "F.Cu") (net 1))
 (segment (start 72 81.48) (end 72 83.6) (width 0.254) (layer "F.Cu") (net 1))
 (segment (start 72 83.6) (end 71.3 84.3) (width 0.254) (layer "F.Cu") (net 1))
 (segment (start 73.6 84.2) (end 73.6 86.9) (width 0.254) (layer "F.Cu") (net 3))
 (segment (start 73 83.6) (end 73.6 84.2) (width 0.254) (layer "F.Cu") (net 3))
 (segment (start 73 81.48) (end 73 83.6) (width 0.254) (layer "F.Cu") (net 3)))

